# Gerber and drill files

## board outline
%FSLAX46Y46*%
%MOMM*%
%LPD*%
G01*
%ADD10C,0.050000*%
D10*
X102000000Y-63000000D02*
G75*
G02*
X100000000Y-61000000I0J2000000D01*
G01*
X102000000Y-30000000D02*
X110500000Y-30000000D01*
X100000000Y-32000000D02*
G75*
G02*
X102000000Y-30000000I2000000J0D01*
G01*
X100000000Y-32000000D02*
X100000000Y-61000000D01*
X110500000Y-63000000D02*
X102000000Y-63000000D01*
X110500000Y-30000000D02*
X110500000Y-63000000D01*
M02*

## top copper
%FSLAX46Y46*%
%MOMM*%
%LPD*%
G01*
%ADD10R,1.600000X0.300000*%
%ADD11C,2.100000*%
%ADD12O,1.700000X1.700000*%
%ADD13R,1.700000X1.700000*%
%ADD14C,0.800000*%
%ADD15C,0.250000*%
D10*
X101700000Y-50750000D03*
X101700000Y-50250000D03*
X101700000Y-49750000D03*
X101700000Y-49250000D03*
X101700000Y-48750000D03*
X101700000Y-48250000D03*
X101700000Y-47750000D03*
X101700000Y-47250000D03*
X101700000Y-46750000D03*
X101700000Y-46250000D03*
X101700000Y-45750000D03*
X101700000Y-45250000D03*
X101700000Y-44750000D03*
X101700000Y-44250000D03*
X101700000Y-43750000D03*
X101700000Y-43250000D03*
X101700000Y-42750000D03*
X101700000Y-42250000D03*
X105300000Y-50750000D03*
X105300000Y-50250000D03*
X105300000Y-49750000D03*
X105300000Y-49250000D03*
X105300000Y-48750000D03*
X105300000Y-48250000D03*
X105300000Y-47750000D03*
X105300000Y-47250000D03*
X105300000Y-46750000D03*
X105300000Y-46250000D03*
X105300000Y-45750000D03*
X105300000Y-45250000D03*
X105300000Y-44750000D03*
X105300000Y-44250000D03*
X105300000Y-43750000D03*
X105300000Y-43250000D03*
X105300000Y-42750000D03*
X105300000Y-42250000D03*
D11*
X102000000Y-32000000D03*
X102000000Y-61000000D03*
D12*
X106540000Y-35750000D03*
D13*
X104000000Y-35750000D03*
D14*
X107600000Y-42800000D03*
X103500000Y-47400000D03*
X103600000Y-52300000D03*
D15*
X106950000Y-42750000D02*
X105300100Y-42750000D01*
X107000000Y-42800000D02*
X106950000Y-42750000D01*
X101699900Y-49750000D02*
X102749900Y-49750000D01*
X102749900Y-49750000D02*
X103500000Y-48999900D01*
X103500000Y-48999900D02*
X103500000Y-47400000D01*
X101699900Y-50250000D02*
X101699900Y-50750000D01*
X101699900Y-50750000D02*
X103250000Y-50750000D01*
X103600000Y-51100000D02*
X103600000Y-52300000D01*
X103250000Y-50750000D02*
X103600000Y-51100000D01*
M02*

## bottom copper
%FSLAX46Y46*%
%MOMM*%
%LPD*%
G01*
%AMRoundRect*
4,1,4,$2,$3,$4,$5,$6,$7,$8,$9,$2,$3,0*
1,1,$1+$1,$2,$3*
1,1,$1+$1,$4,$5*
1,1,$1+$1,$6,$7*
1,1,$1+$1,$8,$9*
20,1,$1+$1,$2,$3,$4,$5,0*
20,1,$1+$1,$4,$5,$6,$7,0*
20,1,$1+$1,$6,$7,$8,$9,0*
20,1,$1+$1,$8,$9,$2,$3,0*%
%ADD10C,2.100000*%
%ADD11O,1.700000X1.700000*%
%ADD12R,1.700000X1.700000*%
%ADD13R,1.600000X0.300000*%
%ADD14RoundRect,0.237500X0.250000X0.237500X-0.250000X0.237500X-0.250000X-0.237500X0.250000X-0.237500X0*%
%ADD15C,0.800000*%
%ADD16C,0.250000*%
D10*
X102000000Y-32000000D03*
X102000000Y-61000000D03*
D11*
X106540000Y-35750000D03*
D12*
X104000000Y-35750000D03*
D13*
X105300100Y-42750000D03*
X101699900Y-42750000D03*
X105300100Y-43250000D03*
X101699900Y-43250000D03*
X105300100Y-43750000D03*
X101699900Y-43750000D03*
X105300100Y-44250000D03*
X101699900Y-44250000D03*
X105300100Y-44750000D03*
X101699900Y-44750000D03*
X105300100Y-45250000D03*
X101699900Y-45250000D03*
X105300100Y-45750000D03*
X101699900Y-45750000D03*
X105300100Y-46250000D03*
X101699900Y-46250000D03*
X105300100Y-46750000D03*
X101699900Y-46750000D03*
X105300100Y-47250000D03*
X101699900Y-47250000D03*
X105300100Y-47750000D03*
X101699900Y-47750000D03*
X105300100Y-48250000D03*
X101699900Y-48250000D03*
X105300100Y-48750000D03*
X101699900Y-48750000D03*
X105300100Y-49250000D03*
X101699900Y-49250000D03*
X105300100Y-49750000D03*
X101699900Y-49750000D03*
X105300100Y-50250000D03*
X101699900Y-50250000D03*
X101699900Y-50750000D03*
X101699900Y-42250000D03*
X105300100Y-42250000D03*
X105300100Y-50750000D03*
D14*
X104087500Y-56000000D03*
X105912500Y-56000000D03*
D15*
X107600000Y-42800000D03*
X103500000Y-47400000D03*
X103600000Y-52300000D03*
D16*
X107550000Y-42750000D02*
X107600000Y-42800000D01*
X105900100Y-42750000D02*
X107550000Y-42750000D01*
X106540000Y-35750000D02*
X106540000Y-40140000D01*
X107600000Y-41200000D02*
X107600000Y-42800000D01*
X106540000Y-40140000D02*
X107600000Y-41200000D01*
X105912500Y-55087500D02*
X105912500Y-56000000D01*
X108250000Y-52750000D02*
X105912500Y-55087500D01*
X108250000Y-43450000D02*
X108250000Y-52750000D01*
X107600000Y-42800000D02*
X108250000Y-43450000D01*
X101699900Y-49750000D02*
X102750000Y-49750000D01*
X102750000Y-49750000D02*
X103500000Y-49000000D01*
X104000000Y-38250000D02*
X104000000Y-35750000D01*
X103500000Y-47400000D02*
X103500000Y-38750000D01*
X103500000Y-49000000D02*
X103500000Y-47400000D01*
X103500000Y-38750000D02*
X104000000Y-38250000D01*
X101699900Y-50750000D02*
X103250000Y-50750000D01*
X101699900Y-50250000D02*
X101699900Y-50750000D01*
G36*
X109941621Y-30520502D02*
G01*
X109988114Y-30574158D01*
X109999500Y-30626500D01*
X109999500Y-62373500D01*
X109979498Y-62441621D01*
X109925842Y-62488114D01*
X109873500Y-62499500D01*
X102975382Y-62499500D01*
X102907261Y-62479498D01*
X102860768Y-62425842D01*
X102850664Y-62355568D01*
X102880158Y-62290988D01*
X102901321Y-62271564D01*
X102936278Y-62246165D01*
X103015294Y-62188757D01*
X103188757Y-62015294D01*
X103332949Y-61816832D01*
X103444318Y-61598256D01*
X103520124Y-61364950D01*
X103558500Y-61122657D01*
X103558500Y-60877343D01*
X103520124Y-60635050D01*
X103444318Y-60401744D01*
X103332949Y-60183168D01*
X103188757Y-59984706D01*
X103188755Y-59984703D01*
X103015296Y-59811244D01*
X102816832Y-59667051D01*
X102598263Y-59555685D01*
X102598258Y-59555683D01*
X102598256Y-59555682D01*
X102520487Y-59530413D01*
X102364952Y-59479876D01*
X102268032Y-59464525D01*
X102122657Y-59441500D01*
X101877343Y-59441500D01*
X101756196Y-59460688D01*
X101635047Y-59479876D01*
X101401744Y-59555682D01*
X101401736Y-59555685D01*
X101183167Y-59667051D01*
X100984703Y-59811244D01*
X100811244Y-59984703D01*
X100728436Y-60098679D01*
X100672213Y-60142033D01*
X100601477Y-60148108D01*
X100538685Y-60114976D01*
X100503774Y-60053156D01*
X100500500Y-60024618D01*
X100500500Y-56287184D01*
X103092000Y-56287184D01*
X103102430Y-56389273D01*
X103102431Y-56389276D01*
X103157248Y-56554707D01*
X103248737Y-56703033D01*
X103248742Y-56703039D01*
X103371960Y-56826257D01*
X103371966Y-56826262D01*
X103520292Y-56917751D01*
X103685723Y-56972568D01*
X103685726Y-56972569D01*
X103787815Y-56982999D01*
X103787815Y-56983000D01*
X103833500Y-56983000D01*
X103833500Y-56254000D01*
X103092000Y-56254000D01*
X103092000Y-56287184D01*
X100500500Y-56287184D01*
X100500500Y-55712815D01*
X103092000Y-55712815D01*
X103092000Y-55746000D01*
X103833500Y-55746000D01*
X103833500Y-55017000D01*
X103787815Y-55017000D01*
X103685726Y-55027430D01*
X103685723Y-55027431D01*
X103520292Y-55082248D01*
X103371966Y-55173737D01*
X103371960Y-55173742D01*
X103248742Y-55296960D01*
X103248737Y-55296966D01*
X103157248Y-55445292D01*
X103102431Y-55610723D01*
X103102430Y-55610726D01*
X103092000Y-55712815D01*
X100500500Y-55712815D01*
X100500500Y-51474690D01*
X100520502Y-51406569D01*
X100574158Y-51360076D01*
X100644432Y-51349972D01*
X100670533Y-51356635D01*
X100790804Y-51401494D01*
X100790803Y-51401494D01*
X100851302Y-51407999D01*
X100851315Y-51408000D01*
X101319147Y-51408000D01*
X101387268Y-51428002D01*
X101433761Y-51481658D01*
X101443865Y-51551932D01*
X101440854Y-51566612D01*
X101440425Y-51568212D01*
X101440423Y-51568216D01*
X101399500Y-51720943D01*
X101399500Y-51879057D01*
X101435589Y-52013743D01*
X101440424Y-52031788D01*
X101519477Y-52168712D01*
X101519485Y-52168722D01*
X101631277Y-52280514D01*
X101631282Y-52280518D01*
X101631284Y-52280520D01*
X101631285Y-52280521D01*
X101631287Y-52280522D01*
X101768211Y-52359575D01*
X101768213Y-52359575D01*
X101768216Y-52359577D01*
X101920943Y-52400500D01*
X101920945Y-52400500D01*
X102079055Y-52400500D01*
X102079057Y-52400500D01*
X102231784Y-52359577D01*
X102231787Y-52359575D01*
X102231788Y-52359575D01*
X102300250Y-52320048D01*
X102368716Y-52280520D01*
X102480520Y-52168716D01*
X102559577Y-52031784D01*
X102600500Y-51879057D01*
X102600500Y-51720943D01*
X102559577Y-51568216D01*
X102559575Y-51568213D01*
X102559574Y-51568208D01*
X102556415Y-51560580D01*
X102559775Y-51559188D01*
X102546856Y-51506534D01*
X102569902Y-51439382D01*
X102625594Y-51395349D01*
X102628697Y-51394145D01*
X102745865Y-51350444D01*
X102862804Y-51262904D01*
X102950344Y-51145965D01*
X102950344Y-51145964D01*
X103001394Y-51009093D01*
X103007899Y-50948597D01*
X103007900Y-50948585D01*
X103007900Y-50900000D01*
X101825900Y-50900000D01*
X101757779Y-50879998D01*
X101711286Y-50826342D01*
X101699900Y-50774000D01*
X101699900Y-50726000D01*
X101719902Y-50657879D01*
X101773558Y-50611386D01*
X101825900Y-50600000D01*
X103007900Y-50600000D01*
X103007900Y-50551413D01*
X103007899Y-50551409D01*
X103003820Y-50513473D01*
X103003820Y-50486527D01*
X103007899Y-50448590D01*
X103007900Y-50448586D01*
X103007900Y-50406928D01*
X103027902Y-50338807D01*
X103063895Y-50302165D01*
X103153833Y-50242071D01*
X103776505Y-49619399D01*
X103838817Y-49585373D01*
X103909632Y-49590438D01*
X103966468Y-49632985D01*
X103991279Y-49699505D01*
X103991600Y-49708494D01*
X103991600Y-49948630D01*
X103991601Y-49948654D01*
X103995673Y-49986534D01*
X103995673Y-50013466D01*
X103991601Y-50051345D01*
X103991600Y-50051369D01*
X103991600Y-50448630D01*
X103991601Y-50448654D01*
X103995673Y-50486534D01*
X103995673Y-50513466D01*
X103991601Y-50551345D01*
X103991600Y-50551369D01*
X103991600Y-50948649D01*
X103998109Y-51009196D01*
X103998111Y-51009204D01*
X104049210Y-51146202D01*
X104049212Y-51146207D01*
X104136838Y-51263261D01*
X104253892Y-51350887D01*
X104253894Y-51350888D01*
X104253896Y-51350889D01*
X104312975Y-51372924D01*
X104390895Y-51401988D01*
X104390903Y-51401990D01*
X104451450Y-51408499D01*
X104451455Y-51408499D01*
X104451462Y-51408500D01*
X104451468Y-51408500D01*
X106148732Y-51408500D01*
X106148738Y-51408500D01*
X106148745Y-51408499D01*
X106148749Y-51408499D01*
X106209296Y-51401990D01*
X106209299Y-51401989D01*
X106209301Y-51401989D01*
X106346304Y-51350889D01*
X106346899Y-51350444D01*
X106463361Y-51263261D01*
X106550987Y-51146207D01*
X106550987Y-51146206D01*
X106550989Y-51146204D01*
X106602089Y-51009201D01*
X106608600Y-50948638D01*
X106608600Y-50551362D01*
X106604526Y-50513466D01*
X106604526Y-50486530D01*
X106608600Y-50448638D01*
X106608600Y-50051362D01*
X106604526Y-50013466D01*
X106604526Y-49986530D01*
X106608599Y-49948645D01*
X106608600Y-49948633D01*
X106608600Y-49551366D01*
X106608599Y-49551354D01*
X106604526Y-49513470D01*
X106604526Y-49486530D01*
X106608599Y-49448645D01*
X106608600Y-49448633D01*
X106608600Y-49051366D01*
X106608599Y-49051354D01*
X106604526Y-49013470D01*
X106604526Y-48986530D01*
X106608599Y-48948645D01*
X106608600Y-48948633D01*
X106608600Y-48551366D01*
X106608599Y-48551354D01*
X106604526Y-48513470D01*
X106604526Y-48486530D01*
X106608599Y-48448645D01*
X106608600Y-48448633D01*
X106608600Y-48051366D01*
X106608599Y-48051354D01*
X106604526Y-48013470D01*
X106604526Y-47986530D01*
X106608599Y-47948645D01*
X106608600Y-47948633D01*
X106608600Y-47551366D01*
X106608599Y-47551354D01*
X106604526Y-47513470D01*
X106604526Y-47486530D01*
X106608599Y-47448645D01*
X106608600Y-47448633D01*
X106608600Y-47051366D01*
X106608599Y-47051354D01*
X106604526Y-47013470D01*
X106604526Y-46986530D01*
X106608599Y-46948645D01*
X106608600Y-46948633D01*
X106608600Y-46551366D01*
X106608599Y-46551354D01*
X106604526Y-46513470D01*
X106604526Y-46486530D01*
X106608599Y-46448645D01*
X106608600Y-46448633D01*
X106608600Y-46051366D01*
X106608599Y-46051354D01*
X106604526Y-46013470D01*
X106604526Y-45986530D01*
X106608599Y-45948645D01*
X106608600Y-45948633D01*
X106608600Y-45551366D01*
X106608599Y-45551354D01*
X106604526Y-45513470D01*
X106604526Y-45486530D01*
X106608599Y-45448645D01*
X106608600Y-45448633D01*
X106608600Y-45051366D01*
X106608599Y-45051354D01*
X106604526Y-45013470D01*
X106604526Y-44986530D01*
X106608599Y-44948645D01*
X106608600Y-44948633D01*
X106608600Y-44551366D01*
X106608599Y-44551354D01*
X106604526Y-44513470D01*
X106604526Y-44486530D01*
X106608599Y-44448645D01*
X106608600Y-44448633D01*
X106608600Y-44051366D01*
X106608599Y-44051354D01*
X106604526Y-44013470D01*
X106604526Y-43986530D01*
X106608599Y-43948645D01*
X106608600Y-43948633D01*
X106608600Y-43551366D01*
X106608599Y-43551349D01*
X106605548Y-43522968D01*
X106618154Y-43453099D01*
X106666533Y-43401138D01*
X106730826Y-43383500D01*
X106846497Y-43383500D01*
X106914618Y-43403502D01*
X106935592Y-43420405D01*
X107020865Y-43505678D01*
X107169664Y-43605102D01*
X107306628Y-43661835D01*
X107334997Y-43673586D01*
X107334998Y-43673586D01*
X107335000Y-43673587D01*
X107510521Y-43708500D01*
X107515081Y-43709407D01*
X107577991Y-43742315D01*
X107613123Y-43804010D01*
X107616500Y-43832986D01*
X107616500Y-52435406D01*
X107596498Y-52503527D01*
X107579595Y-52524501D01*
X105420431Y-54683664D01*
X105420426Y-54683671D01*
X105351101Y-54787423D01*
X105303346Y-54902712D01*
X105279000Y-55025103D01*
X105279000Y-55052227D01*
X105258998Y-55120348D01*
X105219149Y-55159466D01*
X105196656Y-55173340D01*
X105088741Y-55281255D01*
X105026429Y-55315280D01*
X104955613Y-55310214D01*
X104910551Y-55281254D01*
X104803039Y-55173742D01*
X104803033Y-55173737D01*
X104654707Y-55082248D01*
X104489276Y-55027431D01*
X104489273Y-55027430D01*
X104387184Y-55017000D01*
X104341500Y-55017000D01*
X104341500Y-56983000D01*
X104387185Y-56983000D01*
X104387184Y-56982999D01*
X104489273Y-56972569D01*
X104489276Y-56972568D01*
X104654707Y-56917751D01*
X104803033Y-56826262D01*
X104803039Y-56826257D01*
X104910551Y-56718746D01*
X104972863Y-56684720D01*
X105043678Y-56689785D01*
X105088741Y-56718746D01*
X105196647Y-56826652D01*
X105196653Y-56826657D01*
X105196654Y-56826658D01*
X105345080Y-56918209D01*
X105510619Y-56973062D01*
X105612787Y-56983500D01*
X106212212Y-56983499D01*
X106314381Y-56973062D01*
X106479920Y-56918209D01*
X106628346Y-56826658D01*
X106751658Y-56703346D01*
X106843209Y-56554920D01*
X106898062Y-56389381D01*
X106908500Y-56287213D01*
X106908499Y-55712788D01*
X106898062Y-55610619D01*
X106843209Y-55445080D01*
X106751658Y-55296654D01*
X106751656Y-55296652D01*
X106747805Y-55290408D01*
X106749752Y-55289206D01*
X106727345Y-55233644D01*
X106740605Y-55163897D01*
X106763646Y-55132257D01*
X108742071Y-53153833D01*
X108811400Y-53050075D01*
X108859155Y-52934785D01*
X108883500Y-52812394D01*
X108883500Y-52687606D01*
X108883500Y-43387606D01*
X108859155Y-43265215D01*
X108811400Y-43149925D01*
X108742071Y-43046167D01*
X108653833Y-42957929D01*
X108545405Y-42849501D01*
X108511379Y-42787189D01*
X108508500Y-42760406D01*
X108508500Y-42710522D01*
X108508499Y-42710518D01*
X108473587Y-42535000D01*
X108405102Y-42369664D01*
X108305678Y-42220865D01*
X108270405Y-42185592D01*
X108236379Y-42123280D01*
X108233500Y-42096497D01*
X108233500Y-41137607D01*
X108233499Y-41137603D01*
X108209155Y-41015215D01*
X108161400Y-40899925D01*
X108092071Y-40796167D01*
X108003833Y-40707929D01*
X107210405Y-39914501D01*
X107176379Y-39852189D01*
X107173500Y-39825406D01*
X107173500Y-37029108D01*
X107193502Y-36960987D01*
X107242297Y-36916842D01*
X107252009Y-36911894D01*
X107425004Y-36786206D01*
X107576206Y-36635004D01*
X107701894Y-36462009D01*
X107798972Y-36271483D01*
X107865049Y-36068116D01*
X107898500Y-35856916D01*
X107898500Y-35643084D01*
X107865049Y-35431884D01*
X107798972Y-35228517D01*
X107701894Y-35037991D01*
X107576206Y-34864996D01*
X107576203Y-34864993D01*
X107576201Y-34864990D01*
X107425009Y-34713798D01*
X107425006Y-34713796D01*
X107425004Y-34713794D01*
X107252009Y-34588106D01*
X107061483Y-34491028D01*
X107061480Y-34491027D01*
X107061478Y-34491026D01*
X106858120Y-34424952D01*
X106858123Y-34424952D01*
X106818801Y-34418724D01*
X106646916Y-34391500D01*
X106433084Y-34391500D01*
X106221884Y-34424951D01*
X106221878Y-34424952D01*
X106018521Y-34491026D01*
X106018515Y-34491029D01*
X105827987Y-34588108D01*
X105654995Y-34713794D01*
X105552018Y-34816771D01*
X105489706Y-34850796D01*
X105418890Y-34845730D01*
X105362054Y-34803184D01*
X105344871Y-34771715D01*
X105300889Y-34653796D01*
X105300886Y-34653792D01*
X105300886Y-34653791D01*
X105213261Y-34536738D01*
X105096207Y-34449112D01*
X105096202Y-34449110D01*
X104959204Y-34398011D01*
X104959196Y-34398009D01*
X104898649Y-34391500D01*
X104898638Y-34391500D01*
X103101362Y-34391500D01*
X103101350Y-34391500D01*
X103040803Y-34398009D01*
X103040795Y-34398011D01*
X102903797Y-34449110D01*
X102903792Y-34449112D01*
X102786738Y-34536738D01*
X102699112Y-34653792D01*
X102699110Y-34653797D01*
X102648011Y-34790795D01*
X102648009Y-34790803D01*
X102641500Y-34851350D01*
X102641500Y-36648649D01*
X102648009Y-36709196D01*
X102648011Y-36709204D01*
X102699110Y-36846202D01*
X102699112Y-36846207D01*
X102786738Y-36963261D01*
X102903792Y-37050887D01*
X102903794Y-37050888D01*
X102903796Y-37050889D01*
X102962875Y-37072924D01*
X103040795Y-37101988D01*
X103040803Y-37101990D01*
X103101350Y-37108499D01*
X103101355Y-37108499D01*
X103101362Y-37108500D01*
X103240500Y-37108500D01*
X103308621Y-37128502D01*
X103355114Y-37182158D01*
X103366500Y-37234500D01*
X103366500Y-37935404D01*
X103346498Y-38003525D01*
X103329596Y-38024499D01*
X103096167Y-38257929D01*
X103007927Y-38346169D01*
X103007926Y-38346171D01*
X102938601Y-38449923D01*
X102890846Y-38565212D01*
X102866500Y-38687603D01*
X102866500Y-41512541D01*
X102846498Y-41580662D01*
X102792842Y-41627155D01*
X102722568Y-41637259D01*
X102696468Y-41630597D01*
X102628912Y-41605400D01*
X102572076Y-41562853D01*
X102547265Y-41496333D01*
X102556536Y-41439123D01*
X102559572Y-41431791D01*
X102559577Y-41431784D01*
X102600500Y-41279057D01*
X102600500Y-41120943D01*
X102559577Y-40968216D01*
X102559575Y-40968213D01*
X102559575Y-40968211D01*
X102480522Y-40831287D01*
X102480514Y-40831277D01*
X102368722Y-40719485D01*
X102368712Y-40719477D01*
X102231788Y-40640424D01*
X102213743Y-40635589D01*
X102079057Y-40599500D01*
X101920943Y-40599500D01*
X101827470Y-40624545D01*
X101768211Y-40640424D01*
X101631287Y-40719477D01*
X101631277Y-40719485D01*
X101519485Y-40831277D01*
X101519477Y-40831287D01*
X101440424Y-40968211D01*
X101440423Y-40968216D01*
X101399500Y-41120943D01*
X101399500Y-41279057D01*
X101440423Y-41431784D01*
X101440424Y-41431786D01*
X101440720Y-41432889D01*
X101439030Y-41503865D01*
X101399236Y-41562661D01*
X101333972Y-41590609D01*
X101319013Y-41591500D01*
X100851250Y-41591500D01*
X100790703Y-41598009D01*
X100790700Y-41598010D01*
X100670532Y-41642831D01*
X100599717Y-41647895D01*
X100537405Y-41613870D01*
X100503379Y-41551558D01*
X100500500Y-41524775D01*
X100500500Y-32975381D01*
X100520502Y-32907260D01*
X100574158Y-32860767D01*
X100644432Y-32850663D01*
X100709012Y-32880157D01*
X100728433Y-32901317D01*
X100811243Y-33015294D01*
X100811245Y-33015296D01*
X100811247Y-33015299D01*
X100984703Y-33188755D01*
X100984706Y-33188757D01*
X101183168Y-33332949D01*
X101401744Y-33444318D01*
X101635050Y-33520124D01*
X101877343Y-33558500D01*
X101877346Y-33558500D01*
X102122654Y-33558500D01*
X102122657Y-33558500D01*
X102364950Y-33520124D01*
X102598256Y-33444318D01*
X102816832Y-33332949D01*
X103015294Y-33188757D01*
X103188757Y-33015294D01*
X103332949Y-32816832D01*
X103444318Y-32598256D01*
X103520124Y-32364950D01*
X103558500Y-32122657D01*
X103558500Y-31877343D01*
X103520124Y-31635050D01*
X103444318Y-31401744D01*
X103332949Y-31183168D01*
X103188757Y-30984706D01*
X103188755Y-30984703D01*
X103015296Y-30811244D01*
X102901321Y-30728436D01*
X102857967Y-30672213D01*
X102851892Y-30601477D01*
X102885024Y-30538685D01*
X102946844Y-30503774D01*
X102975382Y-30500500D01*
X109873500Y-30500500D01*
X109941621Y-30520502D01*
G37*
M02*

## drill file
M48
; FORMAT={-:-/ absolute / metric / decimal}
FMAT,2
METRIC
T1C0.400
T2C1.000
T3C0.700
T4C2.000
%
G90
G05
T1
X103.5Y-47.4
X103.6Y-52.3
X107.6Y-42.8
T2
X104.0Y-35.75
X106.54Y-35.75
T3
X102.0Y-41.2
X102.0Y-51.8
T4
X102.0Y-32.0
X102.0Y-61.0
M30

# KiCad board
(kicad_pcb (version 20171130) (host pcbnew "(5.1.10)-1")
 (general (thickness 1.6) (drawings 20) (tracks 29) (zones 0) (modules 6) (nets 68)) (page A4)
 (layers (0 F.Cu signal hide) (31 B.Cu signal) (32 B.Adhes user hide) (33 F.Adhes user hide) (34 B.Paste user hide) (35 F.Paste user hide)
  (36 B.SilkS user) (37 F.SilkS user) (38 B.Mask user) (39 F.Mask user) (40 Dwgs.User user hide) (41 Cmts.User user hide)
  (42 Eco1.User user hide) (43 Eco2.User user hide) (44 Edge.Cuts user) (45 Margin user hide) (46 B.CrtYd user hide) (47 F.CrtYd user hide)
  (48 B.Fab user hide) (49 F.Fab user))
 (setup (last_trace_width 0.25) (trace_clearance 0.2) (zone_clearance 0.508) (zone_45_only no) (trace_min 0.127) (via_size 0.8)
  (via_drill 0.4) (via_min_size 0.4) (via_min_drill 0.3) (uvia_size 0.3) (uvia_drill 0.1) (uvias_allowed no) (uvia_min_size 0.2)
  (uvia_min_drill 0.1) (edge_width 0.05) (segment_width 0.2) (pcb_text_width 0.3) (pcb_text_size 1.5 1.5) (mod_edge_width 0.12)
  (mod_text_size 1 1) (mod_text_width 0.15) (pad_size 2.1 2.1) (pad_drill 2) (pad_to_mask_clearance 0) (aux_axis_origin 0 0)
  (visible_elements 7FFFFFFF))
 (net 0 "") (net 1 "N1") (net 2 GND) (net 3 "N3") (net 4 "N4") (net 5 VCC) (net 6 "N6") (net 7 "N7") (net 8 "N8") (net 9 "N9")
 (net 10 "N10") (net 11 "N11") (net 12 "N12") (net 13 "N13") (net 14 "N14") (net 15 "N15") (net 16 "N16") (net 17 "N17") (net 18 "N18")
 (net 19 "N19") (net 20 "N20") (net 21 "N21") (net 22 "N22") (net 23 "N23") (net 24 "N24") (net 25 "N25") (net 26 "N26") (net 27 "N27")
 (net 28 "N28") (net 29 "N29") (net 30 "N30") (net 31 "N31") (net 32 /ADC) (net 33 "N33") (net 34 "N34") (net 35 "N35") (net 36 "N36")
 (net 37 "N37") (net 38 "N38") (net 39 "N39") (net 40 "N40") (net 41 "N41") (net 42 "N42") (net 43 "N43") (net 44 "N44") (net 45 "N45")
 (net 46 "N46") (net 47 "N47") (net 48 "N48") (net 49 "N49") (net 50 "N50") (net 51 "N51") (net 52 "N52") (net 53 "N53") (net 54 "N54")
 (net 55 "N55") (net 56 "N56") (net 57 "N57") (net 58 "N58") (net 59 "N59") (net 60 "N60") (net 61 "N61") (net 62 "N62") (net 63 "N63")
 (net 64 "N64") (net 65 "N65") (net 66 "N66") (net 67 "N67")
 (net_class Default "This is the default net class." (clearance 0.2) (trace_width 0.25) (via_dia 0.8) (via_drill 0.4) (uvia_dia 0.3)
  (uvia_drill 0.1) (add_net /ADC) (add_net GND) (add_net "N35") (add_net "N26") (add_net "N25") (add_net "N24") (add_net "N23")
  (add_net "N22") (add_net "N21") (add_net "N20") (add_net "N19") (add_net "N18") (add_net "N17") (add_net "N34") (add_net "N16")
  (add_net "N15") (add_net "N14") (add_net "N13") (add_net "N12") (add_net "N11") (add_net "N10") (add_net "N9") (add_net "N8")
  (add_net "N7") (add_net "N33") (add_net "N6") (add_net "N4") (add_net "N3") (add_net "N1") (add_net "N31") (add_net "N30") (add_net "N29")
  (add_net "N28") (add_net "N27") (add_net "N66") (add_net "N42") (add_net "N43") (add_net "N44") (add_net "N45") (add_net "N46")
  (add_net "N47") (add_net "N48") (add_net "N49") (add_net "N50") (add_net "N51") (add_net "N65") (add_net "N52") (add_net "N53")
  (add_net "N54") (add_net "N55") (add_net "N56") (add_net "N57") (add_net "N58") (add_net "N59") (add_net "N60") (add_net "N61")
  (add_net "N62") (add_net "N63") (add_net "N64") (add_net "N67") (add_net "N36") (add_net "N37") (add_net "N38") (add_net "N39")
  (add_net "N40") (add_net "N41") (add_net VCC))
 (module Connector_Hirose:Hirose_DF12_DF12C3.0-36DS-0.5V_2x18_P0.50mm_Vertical (layer F.Cu) (at 103.5 46.5 270)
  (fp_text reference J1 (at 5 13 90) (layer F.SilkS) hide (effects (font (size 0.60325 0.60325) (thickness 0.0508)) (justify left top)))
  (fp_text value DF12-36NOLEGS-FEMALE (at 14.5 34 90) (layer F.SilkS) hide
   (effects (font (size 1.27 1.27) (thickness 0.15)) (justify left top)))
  (pad "" smd rect (at 4.25 2 270) (size 0.28 1.2) (layers F.Paste))
  (pad "" smd rect (at 3.75 2 270) (size 0.28 1.2) (layers F.Paste))
  (pad "" smd rect (at 3.25 2 270) (size 0.28 1.2) (layers F.Paste))
  (pad "" smd rect (at 2.75 2 270) (size 0.28 1.2) (layers F.Paste))
  (pad "" smd rect (at 2.25 2 270) (size 0.28 1.2) (layers F.Paste))
  (pad "" smd rect (at 1.75 2 270) (size 0.28 1.2) (layers F.Paste))
  (pad "" smd rect (at 1.25 2 270) (size 0.28 1.2) (layers F.Paste))
  (pad "" smd rect (at 0.75 2 270) (size 0.28 1.2) (layers F.Paste))
  (pad "" smd rect (at 0.25 2 270) (size 0.28 1.2) (layers F.Paste))
  (pad "" smd rect (at -0.25 2 270) (size 0.28 1.2) (layers F.Paste))
  (pad "" smd rect (at -0.75 2 270) (size 0.28 1.2) (layers F.Paste))
  (pad "" smd rect (at -1.25 2 270) (size 0.28 1.2) (layers F.Paste))
  (pad "" smd rect (at -1.75 2 270) (size 0.28 1.2) (layers F.Paste))
  (pad "" smd rect (at -2.25 2 270) (size 0.28 1.2) (layers F.Paste))
  (pad "" smd rect (at -2.75 2 270) (size 0.28 1.2) (layers F.Paste))
  (pad "" smd rect (at -3.25 2 270) (size 0.28 1.2) (layers F.Paste))
  (pad "" smd rect (at -3.75 2 270) (size 0.28 1.2) (layers F.Paste))
  (pad "" smd rect (at -4.25 2 270) (size 0.28 1.2) (layers F.Paste))
  (pad "" smd rect (at 4.25 -2 270) (size 0.28 1.2) (layers F.Paste))
  (pad "" smd rect (at 3.75 -2 270) (size 0.28 1.2) (layers F.Paste))
  (pad "" smd rect (at 3.25 -2 270) (size 0.28 1.2) (layers F.Paste))
  (pad "" smd rect (at 2.75 -2 270) (size 0.28 1.2) (layers F.Paste))
  (pad "" smd rect (at 2.25 -2 270) (size 0.28 1.2) (layers F.Paste))
  (pad "" smd rect (at 1.75 -2 270) (size 0.28 1.2) (layers F.Paste))
  (pad "" smd rect (at 1.25 -2 270) (size 0.28 1.2) (layers F.Paste))
  (pad "" smd rect (at 0.75 -2 270) (size 0.28 1.2) (layers F.Paste))
  (pad "" smd rect (at 0.25 -2 270) (size 0.28 1.2) (layers F.Paste))
  (pad "" smd rect (at -0.25 -2 270) (size 0.28 1.2) (layers F.Paste))
  (pad "" smd rect (at -0.75 -2 270) (size 0.28 1.2) (layers F.Paste))
  (pad "" smd rect (at -1.25 -2 270) (size 0.28 1.2) (layers F.Paste))
  (pad "" smd rect (at -1.75 -2 270) (size 0.28 1.2) (layers F.Paste))
  (pad "" smd rect (at -2.25 -2 270) (size 0.28 1.2) (layers F.Paste))
  (pad "" smd rect (at -2.75 -2 270) (size 0.28 1.2) (layers F.Paste))
  (pad "" smd rect (at -3.25 -2 270) (size 0.28 1.2) (layers F.Paste))
  (pad "" smd rect (at -3.75 -2 270) (size 0.28 1.2) (layers F.Paste))
  (pad "" smd rect (at -4.25 -2 270) (size 0.28 1.2) (layers F.Paste))
  (pad 36 smd rect (at 4.25 1.8 270) (size 0.3 1.6) (layers F.Cu F.Mask) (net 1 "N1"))
  (pad 35 smd rect (at 3.75 1.8 270) (size 0.3 1.6) (layers F.Cu F.Mask) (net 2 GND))
  (pad 34 smd rect (at 3.25 1.8 270) (size 0.3 1.6) (layers F.Cu F.Mask) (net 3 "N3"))
  (pad 33 smd rect (at 2.75 1.8 270) (size 0.3 1.6) (layers F.Cu F.Mask) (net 2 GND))
  (pad 32 smd rect (at 2.25 1.8 270) (size 0.3 1.6) (layers F.Cu F.Mask) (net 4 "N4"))
  (pad 31 smd rect (at 1.75 1.8 270) (size 0.3 1.6) (layers F.Cu F.Mask) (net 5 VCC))
  (pad 30 smd rect (at 1.25 1.8 270) (size 0.3 1.6) (layers F.Cu F.Mask) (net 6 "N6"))
  (pad 29 smd rect (at 0.75 1.8 270) (size 0.3 1.6) (layers F.Cu F.Mask) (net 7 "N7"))
  (pad 28 smd rect (at 0.25 1.8 270) (size 0.3 1.6) (layers F.Cu F.Mask) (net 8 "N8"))
  (pad 27 smd rect (at -0.25 1.8 270) (size 0.3 1.6) (layers F.Cu F.Mask) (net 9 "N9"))
  (pad 26 smd rect (at -0.75 1.8 270) (size 0.3 1.6) (layers F.Cu F.Mask) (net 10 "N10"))
  (pad 25 smd rect (at -1.25 1.8 270) (size 0.3 1.6) (layers F.Cu F.Mask) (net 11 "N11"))
  (pad 24 smd rect (at -1.75 1.8 270) (size 0.3 1.6) (layers F.Cu F.Mask) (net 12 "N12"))
  (pad 23 smd rect (at -2.25 1.8 270) (size 0.3 1.6) (layers F.Cu F.Mask) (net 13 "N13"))
  (pad 22 smd rect (at -2.75 1.8 270) (size 0.3 1.6) (layers F.Cu F.Mask) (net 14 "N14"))
  (pad 21 smd rect (at -3.25 1.8 270) (size 0.3 1.6) (layers F.Cu F.Mask) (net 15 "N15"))
  (pad 20 smd rect (at -3.75 1.8 270) (size 0.3 1.6) (layers F.Cu F.Mask) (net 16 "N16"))
  (pad 19 smd rect (at -4.25 1.8 270) (size 0.3 1.6) (layers F.Cu F.Mask) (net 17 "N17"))
  (pad 18 smd rect (at 4.25 -1.8 270) (size 0.3 1.6) (layers F.Cu F.Mask) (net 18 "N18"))
  (pad 17 smd rect (at 3.75 -1.8 270) (size 0.3 1.6) (layers F.Cu F.Mask) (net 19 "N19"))
  (pad 16 smd rect (at 3.25 -1.8 270) (size 0.3 1.6) (layers F.Cu F.Mask) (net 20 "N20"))
  (pad 15 smd rect (at 2.75 -1.8 270) (size 0.3 1.6) (layers F.Cu F.Mask) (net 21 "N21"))
  (pad 14 smd rect (at 2.25 -1.8 270) (size 0.3 1.6) (layers F.Cu F.Mask) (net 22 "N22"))
  (pad 13 smd rect (at 1.75 -1.8 270) (size 0.3 1.6) (layers F.Cu F.Mask) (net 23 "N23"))
  (pad 12 smd rect (at 1.25 -1.8 270) (size 0.3 1.6) (layers F.Cu F.Mask) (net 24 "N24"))
  (pad 11 smd rect (at 0.75 -1.8 270) (size 0.3 1.6) (layers F.Cu F.Mask) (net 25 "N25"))
  (pad 10 smd rect (at 0.25 -1.8 270) (size 0.3 1.6) (layers F.Cu F.Mask) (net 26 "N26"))
  (pad 9 smd rect (at -0.25 -1.8 270) (size 0.3 1.6) (layers F.Cu F.Mask) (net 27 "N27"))
  (pad 8 smd rect (at -0.75 -1.8 270) (size 0.3 1.6) (layers F.Cu F.Mask) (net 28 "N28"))
  (pad 7 smd rect (at -1.25 -1.8 270) (size 0.3 1.6) (layers F.Cu F.Mask) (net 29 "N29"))
  (pad 6 smd rect (at -1.75 -1.8 270) (size 0.3 1.6) (layers F.Cu F.Mask) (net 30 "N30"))
  (pad 5 smd rect (at -2.25 -1.8 270) (size 0.3 1.6) (layers F.Cu F.Mask) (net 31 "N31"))
  (pad 4 smd rect (at -2.75 -1.8 270) (size 0.3 1.6) (layers F.Cu F.Mask) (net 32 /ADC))
  (pad 3 smd rect (at -3.25 -1.8 270) (size 0.3 1.6) (layers F.Cu F.Mask) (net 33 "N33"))
  (pad 2 smd rect (at -3.75 -1.8 270) (size 0.3 1.6) (layers F.Cu F.Mask) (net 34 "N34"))
  (pad 1 smd rect (at -4.25 -1.8 270) (size 0.3 1.6) (layers F.Cu F.Mask) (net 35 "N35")))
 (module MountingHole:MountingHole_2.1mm (layer F.Cu) (at 102 32)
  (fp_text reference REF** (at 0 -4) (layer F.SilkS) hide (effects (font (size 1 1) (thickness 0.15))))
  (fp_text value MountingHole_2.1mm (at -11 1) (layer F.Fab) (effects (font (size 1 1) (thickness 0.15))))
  (pad "" np_thru_hole circle (at 0 0) (size 2.1 2.1) (drill 2) (layers *.Cu B.Mask)))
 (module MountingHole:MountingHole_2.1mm (layer F.Cu) (at 102 61)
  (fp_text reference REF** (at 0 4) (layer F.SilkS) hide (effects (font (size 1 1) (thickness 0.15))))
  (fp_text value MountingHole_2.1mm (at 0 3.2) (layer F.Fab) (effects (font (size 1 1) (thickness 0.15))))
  (pad "" np_thru_hole circle (at 0 0) (size 2.1 2.1) (drill 2) (layers *.Cu *.Mask)))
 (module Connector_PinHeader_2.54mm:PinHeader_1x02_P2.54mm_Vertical (layer F.Cu) (at 104 35.75 90)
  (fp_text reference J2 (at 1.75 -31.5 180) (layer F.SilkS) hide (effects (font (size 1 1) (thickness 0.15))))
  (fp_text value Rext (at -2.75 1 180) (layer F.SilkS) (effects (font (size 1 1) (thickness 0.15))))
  (pad 2 thru_hole oval (at 0 2.54 90) (size 1.7 1.7) (drill 1) (layers *.Cu *.Mask) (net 32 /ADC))
  (pad 1 thru_hole rect (at 0 0 90) (size 1.7 1.7) (drill 1) (layers *.Cu *.Mask) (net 5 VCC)))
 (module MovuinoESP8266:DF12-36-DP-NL (layer B.Cu) (at 103.5 46.5 270)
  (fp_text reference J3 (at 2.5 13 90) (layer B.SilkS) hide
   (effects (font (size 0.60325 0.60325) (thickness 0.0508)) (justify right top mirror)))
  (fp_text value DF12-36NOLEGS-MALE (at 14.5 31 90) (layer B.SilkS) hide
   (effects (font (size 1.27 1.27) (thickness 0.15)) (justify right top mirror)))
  (pad 3 smd rect (at -3.75 -1.8001 270) (size 0.3 1.6) (layers B.Cu B.Mask) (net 32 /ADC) (solder_mask_margin 0.1016))
  (pad 4 smd rect (at -3.75 1.8001 270) (size 0.3 1.6) (layers B.Cu B.Mask) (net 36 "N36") (solder_mask_margin 0.1016))
  (pad 5 smd rect (at -3.25 -1.8001 270) (size 0.3 1.6) (layers B.Cu B.Mask) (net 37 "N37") (solder_mask_margin 0.1016))
  (pad 6 smd rect (at -3.25 1.8001 270) (size 0.3 1.6) (layers B.Cu B.Mask) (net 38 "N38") (solder_mask_margin 0.1016))
  (pad 7 smd rect (at -2.75 -1.8001 270) (size 0.3 1.6) (layers B.Cu B.Mask) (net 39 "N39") (solder_mask_margin 0.1016))
  (pad 8 smd rect (at -2.75 1.8001 270) (size 0.3 1.6) (layers B.Cu B.Mask) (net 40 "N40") (solder_mask_margin 0.1016))
  (pad 9 smd rect (at -2.25 -1.8001 270) (size 0.3 1.6) (layers B.Cu B.Mask) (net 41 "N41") (solder_mask_margin 0.1016))
  (pad 10 smd rect (at -2.25 1.8001 270) (size 0.3 1.6) (layers B.Cu B.Mask) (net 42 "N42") (solder_mask_margin 0.1016))
  (pad 11 smd rect (at -1.75 -1.8001 270) (size 0.3 1.6) (layers B.Cu B.Mask) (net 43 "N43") (solder_mask_margin 0.1016))
  (pad 12 smd rect (at -1.75 1.8001 270) (size 0.3 1.6) (layers B.Cu B.Mask) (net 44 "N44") (solder_mask_margin 0.1016))
  (pad 13 smd rect (at -1.25 -1.8001 270) (size 0.3 1.6) (layers B.Cu B.Mask) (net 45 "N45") (solder_mask_margin 0.1016))
  (pad 14 smd rect (at -1.25 1.8001 270) (size 0.3 1.6) (layers B.Cu B.Mask) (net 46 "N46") (solder_mask_margin 0.1016))
  (pad 15 smd rect (at -0.75 -1.8001 270) (size 0.3 1.6) (layers B.Cu B.Mask) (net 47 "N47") (solder_mask_margin 0.1016))
  (pad 16 smd rect (at -0.75 1.8001 270) (size 0.3 1.6) (layers B.Cu B.Mask) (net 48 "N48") (solder_mask_margin 0.1016))
  (pad 17 smd rect (at -0.25 -1.8001 270) (size 0.3 1.6) (layers B.Cu B.Mask) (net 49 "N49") (solder_mask_margin 0.1016))
  (pad 18 smd rect (at -0.25 1.8001 270) (size 0.3 1.6) (layers B.Cu B.Mask) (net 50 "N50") (solder_mask_margin 0.1016))
  (pad 19 smd rect (at 0.25 -1.8001 270) (size 0.3 1.6) (layers B.Cu B.Mask) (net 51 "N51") (solder_mask_margin 0.1016))
  (pad 20 smd rect (at 0.25 1.8001 270) (size 0.3 1.6) (layers B.Cu B.Mask) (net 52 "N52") (solder_mask_margin 0.1016))
  (pad 21 smd rect (at 0.75 -1.8001 270) (size 0.3 1.6) (layers B.Cu B.Mask) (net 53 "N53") (solder_mask_margin 0.1016))
  (pad 22 smd rect (at 0.75 1.8001 270) (size 0.3 1.6) (layers B.Cu B.Mask) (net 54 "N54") (solder_mask_margin 0.1016))
  (pad 23 smd rect (at 1.25 -1.8001 270) (size 0.3 1.6) (layers B.Cu B.Mask) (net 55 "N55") (solder_mask_margin 0.1016))
  (pad 24 smd rect (at 1.25 1.8001 270) (size 0.3 1.6) (layers B.Cu B.Mask) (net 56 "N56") (solder_mask_margin 0.1016))
  (pad 25 smd rect (at 1.75 -1.8001 270) (size 0.3 1.6) (layers B.Cu B.Mask) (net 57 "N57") (solder_mask_margin 0.1016))
  (pad 26 smd rect (at 1.75 1.8001 270) (size 0.3 1.6) (layers B.Cu B.Mask) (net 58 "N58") (solder_mask_margin 0.1016))
  (pad 27 smd rect (at 2.25 -1.8001 270) (size 0.3 1.6) (layers B.Cu B.Mask) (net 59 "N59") (solder_mask_margin 0.1016))
  (pad 28 smd rect (at 2.25 1.8001 270) (size 0.3 1.6) (layers B.Cu B.Mask) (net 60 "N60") (solder_mask_margin 0.1016))
  (pad 29 smd rect (at 2.75 -1.8001 270) (size 0.3 1.6) (layers B.Cu B.Mask) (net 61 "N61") (solder_mask_margin 0.1016))
  (pad 30 smd rect (at 2.75 1.8001 270) (size 0.3 1.6) (layers B.Cu B.Mask) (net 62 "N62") (solder_mask_margin 0.1016))
  (pad 31 smd rect (at 3.25 -1.8001 270) (size 0.3 1.6) (layers B.Cu B.Mask) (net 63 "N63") (solder_mask_margin 0.1016))
  (pad 32 smd rect (at 3.25 1.8001 270) (size 0.3 1.6) (layers B.Cu B.Mask) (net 5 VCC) (solder_mask_margin 0.1016))
  (pad 33 smd rect (at 3.75 -1.8001 270) (size 0.3 1.6) (layers B.Cu B.Mask) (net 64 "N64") (solder_mask_margin 0.1016))
  (pad 34 smd rect (at 3.75 1.8001 270) (size 0.3 1.6) (layers B.Cu B.Mask) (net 2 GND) (solder_mask_margin 0.1016))
  (pad 36 smd rect (at 4.25 1.8001 270) (size 0.3 1.6) (layers B.Cu B.Mask) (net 2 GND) (solder_mask_margin 0.1016))
  (pad 2 smd rect (at -4.25 1.8001 270) (size 0.3 1.6) (layers B.Cu B.Mask) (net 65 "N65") (solder_mask_margin 0.1016))
  (pad 1 smd rect (at -4.25 -1.8001 270) (size 0.3 1.6) (layers B.Cu B.Mask) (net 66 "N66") (solder_mask_margin 0.1016))
  (pad 35 smd rect (at 4.25 -1.8001 270) (size 0.3 1.6) (layers B.Cu B.Mask) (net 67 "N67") (solder_mask_margin 0.1016))
  (pad "" np_thru_hole circle (at -5.3 1.5 270) (size 0.7 0.7) (drill 0.7) (layers *.Cu *.Mask))
  (pad "" np_thru_hole circle (at 5.3 1.5 270) (size 0.7 0.7) (drill 0.7) (layers *.Cu *.Mask)))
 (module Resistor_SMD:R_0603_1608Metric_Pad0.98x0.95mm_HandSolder (layer B.Cu) (at 105 56 180)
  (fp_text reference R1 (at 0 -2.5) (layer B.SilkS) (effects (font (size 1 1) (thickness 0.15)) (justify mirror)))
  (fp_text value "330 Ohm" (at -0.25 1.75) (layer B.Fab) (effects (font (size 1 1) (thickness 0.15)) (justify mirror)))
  (pad 2 smd roundrect (at 0.9125 0 180) (size 0.975 0.95) (layers B.Cu B.Paste B.Mask) (roundrect_rratio 0.25) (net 2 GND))
  (pad 1 smd roundrect (at -0.9125 0 180) (size 0.975 0.95) (layers B.Cu B.Paste B.Mask) (roundrect_rratio 0.25) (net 32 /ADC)))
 (gr_arc (start 102 61) (end 100 61) (angle -90) (layer Edge.Cuts) (width 0.05))
 (gr_line (start 102 30) (end 110.5 30) (layer Edge.Cuts) (width 0.05))
 (gr_arc (start 102 32) (end 102 30) (angle -90) (layer Edge.Cuts) (width 0.05))
 (gr_line (start 100 32) (end 100 61) (layer Edge.Cuts) (width 0.05))
 (gr_line (start 110.5 63) (end 102 63) (layer Edge.Cuts) (width 0.05))
 (gr_line (start 110.5 30) (end 110.5 63) (layer Edge.Cuts) (width 0.05))
 (via (at 107.6 42.8) (size 0.8) (drill 0.4) (layers F.Cu B.Cu) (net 32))
 (segment (start 106.95 42.75) (end 105.3001 42.75) (width 0.25) (layer F.Cu) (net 34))
 (segment (start 107 42.8) (end 106.95 42.75) (width 0.25) (layer F.Cu) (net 34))
 (segment (start 107.55 42.75) (end 107.6 42.8) (width 0.25) (layer B.Cu) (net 32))
 (segment (start 105.9001 42.75) (end 107.55 42.75) (width 0.25) (layer B.Cu) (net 32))
 (segment (start 106.54 35.75) (end 106.54 40.14) (width 0.25) (layer B.Cu) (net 32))
 (segment (start 107.6 41.2) (end 107.6 42.8) (width 0.25) (layer B.Cu) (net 32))
 (segment (start 106.54 40.14) (end 107.6 41.2) (width 0.25) (layer B.Cu) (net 32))
 (segment (start 105.9125 55.0875) (end 105.9125 56) (width 0.25) (layer B.Cu) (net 32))
 (segment (start 108.25 52.75) (end 105.9125 55.0875) (width 0.25) (layer B.Cu) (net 32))
 (segment (start 108.25 43.45) (end 108.25 52.75) (width 0.25) (layer B.Cu) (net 32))
 (segment (start 107.6 42.8) (end 108.25 43.45) (width 0.25) (layer B.Cu) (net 32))
 (segment (start 101.6999 49.75) (end 102.75 49.75) (width 0.25) (layer B.Cu) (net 5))
 (segment (start 102.75 49.75) (end 103.5 49) (width 0.25) (layer B.Cu) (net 5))
 (segment (start 104 38.25) (end 104 35.75) (width 0.25) (layer B.Cu) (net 5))
 (segment (start 103.5 47.4) (end 103.5 38.75) (width 0.25) (layer B.Cu) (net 5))
 (segment (start 101.6999 49.75) (end 102.7499 49.75) (width 0.25) (layer F.Cu) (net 5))
 (segment (start 102.7499 49.75) (end 103.5 48.9999) (width 0.25) (layer F.Cu) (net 5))
 (segment (start 103.5 48.9999) (end 103.5 47.4) (width 0.25) (layer F.Cu) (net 5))
 (via (at 103.5 47.4) (size 0.8) (drill 0.4) (layers F.Cu B.Cu) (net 5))
 (segment (start 103.5 49) (end 103.5 47.4) (width 0.25) (layer B.Cu) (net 5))
 (segment (start 103.5 38.75) (end 104 38.25) (width 0.25) (layer B.Cu) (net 5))
 (segment (start 101.6999 50.75) (end 103.25 50.75) (width 0.25) (layer B.Cu) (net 2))
 (segment (start 101.6999 50.25) (end 101.6999 50.75) (width 0.25) (layer B.Cu) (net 2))
 (segment (start 101.6999 50.25) (end 101.6999 50.75) (width 0.25) (layer F.Cu) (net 2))
 (segment (start 101.6999 50.75) (end 103.25 50.75) (width 0.25) (layer F.Cu) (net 2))
 (via (at 103.6 52.3) (size 0.8) (drill 0.4) (layers F.Cu B.Cu) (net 2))
 (segment (start 103.6 51.1) (end 103.6 52.3) (width 0.25) (layer F.Cu) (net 2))
 (segment (start 103.25 50.75) (end 103.6 51.1) (width 0.25) (layer F.Cu) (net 2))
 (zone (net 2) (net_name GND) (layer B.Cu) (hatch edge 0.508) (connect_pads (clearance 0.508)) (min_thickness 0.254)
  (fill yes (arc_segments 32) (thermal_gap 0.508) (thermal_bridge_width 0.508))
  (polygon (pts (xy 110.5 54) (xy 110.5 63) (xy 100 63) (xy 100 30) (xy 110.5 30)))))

